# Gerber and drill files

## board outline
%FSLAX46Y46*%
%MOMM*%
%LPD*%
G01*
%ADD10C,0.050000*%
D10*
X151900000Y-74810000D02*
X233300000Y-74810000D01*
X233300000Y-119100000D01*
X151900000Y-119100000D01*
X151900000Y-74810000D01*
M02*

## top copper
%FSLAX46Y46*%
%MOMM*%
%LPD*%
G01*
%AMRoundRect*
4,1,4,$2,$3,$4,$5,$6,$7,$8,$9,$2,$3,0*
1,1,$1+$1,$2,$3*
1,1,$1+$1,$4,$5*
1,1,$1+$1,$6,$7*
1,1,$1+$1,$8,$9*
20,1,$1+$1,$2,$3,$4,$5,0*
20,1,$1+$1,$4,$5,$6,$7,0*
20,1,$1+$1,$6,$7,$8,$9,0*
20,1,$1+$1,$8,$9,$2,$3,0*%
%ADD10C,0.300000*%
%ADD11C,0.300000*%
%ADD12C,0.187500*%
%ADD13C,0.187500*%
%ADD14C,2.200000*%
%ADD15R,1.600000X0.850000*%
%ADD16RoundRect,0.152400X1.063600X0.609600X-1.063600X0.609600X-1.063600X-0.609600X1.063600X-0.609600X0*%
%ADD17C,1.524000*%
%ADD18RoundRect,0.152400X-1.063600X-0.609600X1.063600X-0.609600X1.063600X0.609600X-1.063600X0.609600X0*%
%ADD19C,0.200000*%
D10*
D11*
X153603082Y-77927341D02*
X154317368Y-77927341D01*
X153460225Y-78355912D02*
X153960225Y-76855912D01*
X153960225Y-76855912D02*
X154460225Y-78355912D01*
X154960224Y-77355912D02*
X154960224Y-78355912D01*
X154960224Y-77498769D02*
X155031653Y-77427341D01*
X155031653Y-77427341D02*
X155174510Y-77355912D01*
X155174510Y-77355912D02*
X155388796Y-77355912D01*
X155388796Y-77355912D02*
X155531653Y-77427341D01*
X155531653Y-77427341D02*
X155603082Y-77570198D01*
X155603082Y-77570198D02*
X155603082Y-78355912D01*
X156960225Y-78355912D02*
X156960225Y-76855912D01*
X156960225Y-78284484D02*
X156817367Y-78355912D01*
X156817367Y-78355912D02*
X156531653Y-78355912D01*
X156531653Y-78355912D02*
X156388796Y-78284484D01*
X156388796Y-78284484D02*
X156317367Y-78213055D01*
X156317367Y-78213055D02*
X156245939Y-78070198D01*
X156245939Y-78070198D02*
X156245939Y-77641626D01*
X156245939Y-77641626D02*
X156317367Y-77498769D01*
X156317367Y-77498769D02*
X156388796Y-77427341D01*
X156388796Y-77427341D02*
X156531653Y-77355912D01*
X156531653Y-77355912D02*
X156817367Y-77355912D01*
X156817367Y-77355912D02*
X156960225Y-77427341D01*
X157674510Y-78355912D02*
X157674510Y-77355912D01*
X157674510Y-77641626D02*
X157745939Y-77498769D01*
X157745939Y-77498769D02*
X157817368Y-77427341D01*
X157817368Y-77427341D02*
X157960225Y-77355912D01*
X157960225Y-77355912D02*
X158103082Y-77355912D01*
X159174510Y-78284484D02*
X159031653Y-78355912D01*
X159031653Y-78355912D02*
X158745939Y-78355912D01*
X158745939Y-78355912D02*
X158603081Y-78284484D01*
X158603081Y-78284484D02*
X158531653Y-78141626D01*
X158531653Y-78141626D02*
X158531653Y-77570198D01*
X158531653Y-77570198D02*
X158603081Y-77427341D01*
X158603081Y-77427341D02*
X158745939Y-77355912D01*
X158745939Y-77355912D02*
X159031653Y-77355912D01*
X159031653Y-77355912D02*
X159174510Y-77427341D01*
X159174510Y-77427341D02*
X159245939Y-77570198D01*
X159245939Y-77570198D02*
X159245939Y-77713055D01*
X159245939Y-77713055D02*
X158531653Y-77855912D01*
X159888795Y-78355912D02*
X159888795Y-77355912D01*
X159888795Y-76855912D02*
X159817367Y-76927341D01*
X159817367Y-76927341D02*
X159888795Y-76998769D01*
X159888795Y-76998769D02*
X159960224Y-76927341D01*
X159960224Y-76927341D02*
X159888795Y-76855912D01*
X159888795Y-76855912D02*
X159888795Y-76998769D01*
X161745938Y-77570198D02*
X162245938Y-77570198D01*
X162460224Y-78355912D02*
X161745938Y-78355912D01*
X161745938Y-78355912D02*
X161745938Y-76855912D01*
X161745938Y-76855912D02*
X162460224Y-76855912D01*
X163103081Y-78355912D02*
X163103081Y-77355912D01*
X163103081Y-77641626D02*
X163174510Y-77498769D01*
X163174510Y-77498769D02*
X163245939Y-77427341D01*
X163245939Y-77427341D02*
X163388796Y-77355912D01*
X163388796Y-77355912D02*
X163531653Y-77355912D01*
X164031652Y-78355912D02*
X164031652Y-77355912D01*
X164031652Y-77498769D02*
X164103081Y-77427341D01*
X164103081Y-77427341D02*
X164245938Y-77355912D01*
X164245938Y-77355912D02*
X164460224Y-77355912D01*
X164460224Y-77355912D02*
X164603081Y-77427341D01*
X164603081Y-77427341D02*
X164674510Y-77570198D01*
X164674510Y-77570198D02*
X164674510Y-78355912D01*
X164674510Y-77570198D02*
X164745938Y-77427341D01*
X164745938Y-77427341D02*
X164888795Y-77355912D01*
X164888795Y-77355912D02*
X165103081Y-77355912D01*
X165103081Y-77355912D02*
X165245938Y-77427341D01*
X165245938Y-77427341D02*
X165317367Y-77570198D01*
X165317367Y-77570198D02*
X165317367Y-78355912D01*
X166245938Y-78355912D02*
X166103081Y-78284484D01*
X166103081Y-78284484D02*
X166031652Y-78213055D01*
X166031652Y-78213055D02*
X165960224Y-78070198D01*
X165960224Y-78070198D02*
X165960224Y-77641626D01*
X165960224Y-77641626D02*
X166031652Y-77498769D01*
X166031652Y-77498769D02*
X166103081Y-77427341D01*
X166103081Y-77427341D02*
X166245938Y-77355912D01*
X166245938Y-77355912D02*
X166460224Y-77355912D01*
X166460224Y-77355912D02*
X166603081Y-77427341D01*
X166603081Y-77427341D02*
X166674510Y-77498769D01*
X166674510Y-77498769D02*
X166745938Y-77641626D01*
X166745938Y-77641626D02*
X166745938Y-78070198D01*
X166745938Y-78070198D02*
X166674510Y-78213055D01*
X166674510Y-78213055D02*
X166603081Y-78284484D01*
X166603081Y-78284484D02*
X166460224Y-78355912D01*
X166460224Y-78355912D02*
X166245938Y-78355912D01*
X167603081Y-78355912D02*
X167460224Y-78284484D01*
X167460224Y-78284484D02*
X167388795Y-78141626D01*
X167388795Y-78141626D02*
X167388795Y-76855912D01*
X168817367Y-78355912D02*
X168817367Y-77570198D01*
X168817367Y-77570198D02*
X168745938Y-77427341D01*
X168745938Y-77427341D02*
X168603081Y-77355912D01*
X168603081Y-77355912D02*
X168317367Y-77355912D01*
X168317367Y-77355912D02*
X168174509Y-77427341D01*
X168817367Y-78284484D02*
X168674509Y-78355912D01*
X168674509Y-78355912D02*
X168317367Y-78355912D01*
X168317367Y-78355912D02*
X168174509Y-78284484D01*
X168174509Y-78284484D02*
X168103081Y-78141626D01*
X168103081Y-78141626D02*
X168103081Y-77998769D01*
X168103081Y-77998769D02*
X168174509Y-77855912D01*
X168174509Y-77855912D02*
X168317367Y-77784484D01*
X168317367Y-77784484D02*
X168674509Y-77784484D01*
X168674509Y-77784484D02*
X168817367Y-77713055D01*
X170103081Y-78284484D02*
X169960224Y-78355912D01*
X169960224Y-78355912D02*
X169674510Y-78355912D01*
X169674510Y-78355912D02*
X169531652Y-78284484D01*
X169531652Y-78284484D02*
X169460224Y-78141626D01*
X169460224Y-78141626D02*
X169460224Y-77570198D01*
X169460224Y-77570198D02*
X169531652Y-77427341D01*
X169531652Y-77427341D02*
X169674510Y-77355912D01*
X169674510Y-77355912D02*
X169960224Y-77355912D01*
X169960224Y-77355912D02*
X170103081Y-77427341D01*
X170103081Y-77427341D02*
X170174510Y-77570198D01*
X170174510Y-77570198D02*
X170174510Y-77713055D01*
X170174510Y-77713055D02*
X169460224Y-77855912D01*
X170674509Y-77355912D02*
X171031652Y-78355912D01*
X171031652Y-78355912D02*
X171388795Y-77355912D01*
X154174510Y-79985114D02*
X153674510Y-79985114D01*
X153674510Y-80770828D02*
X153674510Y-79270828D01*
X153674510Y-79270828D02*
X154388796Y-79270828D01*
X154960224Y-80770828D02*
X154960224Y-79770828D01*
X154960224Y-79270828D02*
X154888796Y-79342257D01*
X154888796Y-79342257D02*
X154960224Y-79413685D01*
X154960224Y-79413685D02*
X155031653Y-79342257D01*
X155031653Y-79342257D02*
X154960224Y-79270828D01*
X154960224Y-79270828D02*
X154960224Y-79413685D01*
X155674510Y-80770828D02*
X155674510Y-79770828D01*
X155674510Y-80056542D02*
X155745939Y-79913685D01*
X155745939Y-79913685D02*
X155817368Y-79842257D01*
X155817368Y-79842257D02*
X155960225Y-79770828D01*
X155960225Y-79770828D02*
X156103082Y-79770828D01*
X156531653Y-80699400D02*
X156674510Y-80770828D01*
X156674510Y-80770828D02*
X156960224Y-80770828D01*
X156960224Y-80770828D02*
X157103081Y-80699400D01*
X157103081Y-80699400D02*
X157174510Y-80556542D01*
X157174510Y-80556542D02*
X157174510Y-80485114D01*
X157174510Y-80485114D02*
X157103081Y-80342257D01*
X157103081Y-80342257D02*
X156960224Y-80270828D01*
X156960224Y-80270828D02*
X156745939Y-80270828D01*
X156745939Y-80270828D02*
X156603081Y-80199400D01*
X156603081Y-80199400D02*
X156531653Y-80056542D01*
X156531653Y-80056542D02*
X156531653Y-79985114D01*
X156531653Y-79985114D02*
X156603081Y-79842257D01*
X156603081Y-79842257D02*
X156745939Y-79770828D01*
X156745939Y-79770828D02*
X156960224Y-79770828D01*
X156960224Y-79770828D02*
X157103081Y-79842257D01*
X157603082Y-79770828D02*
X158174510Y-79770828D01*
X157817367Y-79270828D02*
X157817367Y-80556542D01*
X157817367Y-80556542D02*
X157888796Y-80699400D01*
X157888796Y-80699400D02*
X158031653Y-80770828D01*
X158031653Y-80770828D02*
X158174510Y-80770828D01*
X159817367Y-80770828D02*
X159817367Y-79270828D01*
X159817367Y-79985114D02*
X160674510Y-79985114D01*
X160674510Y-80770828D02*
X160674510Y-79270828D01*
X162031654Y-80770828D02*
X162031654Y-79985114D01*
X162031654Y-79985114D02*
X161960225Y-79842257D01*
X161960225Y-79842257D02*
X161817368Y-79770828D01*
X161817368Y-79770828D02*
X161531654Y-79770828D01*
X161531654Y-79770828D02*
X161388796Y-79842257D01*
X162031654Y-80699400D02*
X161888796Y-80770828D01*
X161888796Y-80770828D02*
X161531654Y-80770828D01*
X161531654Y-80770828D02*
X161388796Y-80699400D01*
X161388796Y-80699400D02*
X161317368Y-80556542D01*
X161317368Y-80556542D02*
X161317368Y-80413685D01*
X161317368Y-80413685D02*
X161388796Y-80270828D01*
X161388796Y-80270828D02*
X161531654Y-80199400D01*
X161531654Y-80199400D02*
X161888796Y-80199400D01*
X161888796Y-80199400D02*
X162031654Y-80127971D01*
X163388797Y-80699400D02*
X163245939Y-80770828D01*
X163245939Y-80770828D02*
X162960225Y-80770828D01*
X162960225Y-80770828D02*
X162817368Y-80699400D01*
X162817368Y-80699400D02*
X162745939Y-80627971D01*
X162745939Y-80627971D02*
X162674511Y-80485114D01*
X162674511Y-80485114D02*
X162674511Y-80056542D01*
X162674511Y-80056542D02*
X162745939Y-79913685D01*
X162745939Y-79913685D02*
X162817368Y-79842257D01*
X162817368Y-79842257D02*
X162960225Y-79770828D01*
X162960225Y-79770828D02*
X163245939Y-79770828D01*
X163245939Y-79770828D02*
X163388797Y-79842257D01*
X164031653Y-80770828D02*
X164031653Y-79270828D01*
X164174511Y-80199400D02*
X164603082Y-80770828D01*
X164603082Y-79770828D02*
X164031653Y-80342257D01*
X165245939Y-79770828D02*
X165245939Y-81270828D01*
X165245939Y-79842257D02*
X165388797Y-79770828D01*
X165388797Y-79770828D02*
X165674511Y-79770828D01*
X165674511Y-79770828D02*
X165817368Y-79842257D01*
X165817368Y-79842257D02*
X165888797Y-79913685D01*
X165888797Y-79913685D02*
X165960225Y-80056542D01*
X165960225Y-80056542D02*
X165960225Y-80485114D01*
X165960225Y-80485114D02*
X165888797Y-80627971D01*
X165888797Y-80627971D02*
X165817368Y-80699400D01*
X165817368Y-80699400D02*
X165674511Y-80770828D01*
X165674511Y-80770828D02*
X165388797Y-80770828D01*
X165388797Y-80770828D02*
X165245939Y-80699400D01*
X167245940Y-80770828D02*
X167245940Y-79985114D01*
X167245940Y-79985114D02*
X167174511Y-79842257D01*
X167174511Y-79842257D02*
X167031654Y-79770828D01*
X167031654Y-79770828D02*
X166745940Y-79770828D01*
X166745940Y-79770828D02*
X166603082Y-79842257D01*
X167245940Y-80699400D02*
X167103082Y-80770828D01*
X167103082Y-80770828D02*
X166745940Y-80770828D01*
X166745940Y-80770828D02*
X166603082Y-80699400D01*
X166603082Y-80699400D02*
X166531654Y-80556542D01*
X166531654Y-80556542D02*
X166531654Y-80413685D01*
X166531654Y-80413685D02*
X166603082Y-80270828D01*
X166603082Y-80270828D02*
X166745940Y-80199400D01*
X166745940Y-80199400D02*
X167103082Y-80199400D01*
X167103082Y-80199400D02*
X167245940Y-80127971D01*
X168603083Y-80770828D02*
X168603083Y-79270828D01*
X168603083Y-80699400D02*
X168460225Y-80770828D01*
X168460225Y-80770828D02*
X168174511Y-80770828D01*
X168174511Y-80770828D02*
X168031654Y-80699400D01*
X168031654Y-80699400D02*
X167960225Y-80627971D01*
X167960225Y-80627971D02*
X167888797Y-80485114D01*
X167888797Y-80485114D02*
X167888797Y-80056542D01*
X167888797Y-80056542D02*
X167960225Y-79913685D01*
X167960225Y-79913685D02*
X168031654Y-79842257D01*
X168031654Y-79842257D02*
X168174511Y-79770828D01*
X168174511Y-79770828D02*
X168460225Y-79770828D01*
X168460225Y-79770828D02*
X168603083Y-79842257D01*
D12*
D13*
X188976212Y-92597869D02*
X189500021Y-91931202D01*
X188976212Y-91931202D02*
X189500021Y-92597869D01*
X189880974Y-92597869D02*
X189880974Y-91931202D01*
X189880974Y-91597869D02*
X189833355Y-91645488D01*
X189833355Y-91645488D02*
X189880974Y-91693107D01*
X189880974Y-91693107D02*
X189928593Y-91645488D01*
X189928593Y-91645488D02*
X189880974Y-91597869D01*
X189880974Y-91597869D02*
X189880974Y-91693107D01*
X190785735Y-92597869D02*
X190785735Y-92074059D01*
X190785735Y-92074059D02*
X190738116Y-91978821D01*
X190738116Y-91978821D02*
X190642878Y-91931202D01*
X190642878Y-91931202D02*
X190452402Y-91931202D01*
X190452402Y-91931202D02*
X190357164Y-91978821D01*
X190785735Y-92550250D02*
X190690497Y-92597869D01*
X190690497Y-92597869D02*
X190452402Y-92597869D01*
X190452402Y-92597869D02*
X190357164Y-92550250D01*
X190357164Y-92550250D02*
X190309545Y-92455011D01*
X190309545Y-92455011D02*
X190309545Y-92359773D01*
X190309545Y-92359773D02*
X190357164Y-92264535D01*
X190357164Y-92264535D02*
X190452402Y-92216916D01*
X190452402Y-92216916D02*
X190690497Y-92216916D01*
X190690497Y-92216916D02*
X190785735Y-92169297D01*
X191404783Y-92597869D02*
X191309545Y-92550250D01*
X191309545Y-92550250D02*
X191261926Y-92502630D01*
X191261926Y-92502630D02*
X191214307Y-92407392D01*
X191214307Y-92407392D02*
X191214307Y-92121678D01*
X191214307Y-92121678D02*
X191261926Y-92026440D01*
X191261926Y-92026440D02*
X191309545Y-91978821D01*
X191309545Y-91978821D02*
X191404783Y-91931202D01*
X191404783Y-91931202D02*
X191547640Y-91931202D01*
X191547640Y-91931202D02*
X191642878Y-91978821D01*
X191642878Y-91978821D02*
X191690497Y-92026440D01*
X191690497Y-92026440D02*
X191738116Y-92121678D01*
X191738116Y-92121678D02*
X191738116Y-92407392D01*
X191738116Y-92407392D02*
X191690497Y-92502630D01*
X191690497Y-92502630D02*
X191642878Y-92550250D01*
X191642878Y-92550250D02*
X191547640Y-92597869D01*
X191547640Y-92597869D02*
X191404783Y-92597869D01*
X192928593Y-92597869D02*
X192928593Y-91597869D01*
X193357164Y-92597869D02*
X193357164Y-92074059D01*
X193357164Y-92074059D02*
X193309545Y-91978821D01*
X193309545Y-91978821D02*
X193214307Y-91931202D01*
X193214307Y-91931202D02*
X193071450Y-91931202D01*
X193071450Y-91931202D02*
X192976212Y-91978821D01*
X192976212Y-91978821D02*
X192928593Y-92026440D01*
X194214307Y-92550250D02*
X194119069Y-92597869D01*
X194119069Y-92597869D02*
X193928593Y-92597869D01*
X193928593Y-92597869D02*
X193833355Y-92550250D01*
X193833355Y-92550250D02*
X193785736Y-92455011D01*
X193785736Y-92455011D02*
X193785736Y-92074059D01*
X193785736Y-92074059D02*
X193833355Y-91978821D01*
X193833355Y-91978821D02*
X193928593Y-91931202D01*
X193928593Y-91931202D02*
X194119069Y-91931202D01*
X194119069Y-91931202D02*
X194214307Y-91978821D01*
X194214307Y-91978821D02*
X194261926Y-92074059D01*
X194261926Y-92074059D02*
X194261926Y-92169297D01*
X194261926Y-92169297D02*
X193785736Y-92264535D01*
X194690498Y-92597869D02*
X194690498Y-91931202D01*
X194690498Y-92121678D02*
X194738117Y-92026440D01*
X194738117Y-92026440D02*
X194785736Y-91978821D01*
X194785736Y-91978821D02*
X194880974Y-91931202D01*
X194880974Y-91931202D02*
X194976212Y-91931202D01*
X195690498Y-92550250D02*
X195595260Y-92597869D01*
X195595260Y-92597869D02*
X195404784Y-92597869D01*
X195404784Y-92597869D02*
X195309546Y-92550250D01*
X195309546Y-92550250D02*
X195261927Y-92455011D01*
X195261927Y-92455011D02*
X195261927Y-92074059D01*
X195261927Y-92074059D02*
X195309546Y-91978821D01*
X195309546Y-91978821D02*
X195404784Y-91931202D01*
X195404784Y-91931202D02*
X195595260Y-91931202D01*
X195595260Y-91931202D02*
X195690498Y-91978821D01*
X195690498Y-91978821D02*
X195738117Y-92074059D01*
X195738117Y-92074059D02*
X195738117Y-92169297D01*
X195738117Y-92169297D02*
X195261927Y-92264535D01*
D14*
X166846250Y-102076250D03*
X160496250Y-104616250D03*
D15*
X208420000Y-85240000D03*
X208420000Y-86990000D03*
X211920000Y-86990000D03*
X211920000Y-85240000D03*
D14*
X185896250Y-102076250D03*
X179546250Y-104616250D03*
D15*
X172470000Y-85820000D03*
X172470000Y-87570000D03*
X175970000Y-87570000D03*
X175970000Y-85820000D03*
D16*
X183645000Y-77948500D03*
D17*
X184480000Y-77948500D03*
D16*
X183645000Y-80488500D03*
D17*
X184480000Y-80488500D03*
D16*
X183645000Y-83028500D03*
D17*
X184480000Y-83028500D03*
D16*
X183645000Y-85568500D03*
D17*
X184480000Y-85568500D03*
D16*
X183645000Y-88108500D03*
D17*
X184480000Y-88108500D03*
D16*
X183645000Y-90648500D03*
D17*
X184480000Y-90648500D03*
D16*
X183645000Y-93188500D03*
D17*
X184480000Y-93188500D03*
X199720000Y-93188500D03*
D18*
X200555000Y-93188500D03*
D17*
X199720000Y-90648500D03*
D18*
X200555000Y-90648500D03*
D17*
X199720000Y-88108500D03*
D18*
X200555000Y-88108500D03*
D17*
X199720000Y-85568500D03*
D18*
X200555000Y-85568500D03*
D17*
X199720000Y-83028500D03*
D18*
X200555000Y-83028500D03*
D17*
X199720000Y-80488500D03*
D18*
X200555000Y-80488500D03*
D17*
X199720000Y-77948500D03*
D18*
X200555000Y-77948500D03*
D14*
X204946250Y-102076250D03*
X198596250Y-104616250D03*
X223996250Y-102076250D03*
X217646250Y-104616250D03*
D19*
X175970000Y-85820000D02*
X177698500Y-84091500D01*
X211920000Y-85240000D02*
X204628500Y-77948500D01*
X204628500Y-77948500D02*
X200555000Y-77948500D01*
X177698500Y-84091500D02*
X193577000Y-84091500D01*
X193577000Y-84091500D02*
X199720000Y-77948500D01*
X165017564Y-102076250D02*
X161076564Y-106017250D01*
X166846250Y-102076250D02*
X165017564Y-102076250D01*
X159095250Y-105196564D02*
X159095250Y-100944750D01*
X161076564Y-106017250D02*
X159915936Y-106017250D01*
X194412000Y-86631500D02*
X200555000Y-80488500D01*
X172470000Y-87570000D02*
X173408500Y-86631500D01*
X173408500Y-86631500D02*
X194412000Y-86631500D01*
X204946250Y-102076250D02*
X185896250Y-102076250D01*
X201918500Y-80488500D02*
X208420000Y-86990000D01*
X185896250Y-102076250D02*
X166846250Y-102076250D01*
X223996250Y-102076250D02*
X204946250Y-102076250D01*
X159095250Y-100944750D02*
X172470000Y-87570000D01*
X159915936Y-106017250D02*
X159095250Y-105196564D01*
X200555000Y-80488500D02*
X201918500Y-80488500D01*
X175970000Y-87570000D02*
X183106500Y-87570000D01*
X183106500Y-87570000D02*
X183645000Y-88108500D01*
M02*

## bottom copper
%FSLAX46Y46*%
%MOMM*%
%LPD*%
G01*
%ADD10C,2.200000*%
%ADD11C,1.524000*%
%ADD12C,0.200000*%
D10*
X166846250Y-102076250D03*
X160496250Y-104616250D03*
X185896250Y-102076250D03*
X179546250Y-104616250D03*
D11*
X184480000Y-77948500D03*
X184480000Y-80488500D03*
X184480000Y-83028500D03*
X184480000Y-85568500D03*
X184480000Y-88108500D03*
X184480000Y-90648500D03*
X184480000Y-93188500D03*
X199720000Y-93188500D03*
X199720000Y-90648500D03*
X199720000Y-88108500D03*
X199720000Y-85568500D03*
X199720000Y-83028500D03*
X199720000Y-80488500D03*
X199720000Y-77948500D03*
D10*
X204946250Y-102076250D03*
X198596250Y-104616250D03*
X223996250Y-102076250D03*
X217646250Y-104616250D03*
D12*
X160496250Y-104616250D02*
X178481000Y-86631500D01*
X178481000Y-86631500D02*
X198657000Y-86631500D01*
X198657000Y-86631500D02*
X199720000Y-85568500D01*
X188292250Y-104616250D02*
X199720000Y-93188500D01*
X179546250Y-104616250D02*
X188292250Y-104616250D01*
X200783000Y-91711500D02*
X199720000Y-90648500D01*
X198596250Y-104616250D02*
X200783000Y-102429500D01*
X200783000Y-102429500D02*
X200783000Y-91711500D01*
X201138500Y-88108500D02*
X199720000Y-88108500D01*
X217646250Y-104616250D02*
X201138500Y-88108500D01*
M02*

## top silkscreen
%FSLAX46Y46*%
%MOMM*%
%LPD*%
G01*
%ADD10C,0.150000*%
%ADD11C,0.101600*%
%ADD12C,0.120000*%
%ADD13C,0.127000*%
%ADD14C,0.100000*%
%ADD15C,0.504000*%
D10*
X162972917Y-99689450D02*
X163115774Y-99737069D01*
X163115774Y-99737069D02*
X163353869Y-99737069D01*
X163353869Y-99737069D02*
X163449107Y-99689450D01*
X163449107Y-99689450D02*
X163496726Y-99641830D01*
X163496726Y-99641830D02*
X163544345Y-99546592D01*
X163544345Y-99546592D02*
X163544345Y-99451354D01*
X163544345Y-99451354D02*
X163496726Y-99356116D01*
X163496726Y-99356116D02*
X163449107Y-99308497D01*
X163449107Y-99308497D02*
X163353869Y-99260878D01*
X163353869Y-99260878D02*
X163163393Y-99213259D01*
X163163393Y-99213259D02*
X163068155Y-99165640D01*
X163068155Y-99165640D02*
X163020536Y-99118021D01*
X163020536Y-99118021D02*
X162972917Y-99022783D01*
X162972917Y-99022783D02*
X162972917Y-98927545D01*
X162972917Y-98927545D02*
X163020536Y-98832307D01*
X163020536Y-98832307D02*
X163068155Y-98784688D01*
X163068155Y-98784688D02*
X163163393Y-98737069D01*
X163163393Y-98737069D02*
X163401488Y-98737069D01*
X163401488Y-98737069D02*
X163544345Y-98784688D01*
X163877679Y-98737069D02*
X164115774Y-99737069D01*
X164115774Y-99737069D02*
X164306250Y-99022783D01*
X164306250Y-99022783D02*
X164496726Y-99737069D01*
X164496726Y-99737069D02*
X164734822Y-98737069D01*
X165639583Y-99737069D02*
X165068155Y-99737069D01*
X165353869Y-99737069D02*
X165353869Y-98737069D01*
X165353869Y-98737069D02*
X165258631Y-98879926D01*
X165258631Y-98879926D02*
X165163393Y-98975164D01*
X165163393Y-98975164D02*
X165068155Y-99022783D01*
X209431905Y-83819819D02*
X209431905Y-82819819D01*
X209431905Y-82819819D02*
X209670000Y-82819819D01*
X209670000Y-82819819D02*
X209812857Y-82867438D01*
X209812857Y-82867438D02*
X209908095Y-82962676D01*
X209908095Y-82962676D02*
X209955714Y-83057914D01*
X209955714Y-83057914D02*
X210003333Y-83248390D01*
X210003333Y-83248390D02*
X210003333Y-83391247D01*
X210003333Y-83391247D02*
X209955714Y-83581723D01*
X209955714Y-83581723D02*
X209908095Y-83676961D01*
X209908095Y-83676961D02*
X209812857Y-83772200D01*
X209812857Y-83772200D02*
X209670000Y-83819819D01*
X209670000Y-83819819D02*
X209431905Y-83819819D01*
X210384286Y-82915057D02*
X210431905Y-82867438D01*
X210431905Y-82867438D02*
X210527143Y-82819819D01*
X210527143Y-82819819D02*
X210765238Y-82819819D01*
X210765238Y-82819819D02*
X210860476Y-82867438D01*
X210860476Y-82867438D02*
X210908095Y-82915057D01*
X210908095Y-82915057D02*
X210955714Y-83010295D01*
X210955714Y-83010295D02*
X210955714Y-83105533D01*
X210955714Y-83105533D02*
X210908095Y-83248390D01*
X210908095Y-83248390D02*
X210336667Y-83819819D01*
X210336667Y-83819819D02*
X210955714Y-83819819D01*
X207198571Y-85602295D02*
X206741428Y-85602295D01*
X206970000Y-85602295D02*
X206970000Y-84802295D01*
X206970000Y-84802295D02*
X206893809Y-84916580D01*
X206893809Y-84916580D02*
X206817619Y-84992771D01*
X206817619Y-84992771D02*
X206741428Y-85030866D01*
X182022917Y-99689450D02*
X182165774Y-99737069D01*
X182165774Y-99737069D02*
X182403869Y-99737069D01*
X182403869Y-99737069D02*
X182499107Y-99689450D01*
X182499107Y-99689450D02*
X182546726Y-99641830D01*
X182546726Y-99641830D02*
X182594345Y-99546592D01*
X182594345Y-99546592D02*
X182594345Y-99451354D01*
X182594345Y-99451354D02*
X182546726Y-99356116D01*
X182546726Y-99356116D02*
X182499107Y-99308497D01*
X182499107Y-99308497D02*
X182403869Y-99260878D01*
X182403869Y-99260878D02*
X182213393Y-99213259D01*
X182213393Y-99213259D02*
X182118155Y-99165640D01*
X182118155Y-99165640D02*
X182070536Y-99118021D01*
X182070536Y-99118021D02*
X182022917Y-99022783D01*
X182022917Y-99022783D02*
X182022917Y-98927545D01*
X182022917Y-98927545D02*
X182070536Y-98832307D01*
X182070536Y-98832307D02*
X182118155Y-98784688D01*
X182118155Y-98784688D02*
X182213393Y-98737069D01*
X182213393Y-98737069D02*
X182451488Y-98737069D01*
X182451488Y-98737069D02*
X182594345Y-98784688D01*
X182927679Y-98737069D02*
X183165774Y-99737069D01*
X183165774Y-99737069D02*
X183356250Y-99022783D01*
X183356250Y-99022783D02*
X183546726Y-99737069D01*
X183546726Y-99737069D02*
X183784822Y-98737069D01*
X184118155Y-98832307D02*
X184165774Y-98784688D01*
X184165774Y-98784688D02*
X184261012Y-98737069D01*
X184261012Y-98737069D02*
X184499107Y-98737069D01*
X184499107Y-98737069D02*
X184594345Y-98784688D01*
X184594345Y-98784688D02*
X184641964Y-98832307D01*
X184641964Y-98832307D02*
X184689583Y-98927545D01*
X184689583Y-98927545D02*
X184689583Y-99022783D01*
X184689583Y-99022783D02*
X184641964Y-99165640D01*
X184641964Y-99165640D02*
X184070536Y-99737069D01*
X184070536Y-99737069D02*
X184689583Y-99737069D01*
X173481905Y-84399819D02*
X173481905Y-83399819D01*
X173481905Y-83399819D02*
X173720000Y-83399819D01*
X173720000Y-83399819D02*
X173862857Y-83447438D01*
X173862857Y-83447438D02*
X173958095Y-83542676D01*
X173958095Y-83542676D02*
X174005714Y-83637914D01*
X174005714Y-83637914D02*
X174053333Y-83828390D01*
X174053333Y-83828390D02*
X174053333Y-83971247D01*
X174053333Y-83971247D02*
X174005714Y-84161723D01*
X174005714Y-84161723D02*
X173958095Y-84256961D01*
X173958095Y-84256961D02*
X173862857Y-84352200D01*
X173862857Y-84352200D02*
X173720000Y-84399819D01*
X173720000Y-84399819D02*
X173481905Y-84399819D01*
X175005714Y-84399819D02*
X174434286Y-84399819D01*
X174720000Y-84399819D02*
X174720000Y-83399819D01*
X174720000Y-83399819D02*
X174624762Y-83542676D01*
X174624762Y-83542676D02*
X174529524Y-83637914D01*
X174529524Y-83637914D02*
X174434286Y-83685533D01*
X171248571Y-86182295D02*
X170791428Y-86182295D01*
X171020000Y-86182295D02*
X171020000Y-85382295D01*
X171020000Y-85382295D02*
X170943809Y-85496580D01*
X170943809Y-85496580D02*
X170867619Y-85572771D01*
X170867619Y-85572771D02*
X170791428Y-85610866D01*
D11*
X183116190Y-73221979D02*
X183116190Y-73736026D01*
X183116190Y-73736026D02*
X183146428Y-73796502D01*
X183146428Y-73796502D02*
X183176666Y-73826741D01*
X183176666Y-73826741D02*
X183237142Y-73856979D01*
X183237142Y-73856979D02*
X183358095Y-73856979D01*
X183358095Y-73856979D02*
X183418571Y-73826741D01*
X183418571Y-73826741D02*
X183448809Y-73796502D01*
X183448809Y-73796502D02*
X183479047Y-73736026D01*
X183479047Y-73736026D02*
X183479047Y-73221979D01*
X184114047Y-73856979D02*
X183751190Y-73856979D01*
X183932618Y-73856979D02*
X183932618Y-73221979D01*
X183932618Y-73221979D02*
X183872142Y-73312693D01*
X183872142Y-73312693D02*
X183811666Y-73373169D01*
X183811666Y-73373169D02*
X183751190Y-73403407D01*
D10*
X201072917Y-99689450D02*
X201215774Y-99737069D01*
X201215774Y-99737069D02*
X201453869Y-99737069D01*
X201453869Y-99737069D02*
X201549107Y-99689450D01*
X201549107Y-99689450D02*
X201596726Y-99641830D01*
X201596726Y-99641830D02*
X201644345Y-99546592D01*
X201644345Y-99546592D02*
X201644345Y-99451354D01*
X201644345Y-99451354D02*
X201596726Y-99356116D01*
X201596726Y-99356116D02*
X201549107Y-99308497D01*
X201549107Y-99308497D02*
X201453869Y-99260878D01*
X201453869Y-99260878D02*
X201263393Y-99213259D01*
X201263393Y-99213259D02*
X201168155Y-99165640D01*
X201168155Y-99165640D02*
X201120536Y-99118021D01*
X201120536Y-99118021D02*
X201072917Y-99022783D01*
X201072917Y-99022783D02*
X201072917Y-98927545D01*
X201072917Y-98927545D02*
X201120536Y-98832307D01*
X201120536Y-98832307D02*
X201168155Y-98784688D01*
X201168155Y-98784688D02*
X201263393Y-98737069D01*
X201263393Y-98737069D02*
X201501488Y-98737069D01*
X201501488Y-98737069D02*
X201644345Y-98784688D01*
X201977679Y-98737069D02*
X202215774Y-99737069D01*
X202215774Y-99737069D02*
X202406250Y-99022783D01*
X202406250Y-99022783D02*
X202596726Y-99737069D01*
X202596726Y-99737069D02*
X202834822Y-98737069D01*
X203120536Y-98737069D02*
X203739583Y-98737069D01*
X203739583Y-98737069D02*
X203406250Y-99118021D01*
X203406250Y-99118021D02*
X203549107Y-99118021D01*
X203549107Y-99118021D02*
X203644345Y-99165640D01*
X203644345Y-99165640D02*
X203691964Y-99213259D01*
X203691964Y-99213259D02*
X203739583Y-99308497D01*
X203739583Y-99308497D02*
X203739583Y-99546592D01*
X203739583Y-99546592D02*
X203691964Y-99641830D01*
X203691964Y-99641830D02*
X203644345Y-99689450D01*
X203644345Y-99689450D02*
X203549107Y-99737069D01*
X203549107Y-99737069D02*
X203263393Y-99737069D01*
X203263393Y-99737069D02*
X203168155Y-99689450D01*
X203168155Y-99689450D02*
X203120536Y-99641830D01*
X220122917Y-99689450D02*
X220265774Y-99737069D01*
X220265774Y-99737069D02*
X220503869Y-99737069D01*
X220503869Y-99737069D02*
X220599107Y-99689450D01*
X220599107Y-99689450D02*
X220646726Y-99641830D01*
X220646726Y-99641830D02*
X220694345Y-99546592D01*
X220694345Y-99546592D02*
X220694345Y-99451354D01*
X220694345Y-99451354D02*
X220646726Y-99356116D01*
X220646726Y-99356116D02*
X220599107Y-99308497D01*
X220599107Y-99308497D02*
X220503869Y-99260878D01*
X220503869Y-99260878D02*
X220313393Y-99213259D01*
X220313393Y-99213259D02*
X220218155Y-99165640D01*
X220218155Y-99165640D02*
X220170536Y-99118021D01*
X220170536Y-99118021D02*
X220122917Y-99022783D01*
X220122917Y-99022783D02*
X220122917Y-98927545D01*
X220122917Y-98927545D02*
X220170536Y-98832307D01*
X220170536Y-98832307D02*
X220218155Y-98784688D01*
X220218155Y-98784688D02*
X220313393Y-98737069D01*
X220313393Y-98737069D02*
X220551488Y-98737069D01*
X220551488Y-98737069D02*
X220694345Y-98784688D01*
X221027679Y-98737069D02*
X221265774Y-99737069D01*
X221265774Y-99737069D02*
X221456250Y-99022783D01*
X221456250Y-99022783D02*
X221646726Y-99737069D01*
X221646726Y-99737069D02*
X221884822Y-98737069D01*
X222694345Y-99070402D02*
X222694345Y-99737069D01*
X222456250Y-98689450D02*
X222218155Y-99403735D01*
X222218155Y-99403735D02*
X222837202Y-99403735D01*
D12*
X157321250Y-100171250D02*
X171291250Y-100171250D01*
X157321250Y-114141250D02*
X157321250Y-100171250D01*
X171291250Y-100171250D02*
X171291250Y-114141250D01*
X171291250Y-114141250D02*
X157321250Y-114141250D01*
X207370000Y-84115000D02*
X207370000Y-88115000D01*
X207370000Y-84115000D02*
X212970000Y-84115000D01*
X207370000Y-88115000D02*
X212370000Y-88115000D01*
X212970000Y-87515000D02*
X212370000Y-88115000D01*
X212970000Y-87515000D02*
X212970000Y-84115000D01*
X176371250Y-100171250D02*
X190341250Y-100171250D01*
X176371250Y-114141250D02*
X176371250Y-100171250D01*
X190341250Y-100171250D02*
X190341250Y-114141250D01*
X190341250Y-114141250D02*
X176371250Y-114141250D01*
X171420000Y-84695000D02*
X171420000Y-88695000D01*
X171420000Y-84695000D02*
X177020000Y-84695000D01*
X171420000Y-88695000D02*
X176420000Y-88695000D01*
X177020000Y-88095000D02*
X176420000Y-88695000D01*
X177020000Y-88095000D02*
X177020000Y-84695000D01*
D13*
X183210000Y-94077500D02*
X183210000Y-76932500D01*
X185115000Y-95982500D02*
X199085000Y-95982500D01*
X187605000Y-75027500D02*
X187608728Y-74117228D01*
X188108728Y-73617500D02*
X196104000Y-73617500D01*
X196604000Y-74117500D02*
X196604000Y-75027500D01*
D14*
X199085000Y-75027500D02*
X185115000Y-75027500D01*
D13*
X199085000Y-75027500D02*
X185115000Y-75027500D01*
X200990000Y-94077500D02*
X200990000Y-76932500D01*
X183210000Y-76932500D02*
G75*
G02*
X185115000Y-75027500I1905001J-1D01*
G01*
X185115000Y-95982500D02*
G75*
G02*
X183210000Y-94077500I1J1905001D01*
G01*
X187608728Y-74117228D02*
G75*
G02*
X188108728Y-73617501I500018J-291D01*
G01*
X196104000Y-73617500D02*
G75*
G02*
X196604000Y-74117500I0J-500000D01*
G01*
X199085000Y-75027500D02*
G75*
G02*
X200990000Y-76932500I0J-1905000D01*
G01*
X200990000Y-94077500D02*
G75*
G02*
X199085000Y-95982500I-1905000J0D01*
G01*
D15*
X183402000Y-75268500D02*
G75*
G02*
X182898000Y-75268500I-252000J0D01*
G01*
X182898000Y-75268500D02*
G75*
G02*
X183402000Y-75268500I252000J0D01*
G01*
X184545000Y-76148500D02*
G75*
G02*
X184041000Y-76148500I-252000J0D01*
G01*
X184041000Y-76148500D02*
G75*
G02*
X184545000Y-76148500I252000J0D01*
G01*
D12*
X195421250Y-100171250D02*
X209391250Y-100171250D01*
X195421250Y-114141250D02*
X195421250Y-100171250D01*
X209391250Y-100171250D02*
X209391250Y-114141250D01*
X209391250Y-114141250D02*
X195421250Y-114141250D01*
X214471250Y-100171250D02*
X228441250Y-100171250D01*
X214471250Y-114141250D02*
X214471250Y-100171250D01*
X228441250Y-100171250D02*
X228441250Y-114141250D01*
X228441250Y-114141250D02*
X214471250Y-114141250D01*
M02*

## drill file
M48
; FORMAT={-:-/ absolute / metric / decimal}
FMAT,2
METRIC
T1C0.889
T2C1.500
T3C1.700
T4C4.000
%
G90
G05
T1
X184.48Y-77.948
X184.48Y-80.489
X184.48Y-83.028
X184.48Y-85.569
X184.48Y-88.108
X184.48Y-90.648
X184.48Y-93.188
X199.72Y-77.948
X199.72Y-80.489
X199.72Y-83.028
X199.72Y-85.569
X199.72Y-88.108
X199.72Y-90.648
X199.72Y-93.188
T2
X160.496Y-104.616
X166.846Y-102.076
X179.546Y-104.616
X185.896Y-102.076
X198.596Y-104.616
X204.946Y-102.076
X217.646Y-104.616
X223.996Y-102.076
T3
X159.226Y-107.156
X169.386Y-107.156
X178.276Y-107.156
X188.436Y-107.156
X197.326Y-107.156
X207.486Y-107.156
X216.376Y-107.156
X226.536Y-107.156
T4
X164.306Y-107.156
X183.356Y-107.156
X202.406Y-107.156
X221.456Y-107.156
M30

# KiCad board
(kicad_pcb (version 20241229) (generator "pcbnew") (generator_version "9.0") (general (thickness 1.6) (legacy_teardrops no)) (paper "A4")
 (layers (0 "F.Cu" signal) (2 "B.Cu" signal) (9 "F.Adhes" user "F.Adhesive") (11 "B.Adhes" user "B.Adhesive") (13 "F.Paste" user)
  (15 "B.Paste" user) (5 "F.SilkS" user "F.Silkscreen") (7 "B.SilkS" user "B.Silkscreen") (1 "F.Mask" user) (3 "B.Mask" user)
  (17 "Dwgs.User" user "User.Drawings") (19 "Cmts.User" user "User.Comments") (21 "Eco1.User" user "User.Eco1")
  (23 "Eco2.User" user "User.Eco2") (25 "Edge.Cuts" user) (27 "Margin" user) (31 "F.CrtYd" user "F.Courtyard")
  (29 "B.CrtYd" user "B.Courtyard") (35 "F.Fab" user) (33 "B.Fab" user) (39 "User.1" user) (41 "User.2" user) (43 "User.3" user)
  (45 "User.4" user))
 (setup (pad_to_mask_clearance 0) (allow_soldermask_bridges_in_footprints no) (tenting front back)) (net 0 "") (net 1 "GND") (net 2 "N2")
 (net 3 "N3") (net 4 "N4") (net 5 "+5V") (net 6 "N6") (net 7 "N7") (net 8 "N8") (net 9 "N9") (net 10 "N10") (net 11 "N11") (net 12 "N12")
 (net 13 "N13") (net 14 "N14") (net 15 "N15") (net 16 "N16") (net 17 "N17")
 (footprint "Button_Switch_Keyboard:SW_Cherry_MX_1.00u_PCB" (layer "F.Cu") (at 166.84625 102.07625)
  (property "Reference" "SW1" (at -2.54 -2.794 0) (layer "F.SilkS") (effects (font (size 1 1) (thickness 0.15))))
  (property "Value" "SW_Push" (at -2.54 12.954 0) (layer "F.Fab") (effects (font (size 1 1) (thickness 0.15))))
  (fp_line (start -9.525 -1.905) (end 4.445 -1.905) (stroke (width 0.12) (type solid)) (layer "F.SilkS"))
  (fp_line (start -9.525 12.065) (end -9.525 -1.905) (stroke (width 0.12) (type solid)) (layer "F.SilkS"))
  (fp_line (start 4.445 -1.905) (end 4.445 12.065) (stroke (width 0.12) (type solid)) (layer "F.SilkS"))
  (fp_line (start 4.445 12.065) (end -9.525 12.065) (stroke (width 0.12) (type solid)) (layer "F.SilkS"))
  (pad "" np_thru_hole circle (at -7.62 5.08) (size 1.7 1.7) (drill 1.7) (layers "*.Cu" "*.Mask"))
  (pad "" np_thru_hole circle (at -2.54 5.08) (size 4 4) (drill 4) (layers "*.Cu" "*.Mask"))
  (pad "" np_thru_hole circle (at 2.54 5.08) (size 1.7 1.7) (drill 1.7) (layers "*.Cu" "*.Mask"))
  (pad "1" thru_hole circle (at 0 0) (size 2.2 2.2) (drill 1.5) (layers "*.Cu" "*.Mask") (remove_unused_layers no) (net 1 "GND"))
  (pad "2" thru_hole circle (at -6.35 2.54) (size 2.2 2.2) (drill 1.5) (layers "*.Cu" "*.Mask") (remove_unused_layers no) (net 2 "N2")))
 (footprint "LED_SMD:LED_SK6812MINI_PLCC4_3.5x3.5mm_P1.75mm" (layer "F.Cu") (at 210.17 86.115)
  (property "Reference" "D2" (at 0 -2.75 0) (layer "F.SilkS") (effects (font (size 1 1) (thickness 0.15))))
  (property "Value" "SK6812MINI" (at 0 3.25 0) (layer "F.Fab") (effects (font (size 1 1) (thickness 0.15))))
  (fp_line (start -2.8 -2) (end -2.8 2) (stroke (width 0.12) (type default)) (layer "F.SilkS"))
  (fp_line (start -2.8 -2) (end 2.8 -2) (stroke (width 0.12) (type solid)) (layer "F.SilkS"))
  (fp_line (start -2.8 2) (end 2.2 2) (stroke (width 0.12) (type solid)) (layer "F.SilkS"))
  (fp_line (start 2.8 1.4) (end 2.2 2) (stroke (width 0.12) (type default)) (layer "F.SilkS"))
  (fp_line (start 2.8 1.4) (end 2.8 -2) (stroke (width 0.12) (type solid)) (layer "F.SilkS"))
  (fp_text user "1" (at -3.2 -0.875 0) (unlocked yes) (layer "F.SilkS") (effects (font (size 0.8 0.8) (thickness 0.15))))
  (pad "1" smd rect (at -1.75 -0.875) (size 1.6 0.85) (layers "F.Cu" "F.Mask" "F.Paste") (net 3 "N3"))
  (pad "2" smd rect (at -1.75 0.875) (size 1.6 0.85) (layers "F.Cu" "F.Mask" "F.Paste") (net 1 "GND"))
  (pad "3" smd rect (at 1.75 0.875) (size 1.6 0.85) (layers "F.Cu" "F.Mask" "F.Paste") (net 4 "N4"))
  (pad "4" smd rect (at 1.75 -0.875) (size 1.6 0.85) (layers "F.Cu" "F.Mask" "F.Paste") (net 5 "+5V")))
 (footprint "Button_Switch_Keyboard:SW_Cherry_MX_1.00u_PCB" (layer "F.Cu") (at 185.89625 102.07625)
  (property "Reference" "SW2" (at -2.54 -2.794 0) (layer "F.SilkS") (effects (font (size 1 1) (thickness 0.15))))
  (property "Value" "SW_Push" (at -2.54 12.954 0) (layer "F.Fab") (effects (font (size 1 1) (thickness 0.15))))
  (fp_line (start -9.525 -1.905) (end 4.445 -1.905) (stroke (width 0.12) (type solid)) (layer "F.SilkS"))
  (fp_line (start -9.525 12.065) (end -9.525 -1.905) (stroke (width 0.12) (type solid)) (layer "F.SilkS"))
  (fp_line (start 4.445 -1.905) (end 4.445 12.065) (stroke (width 0.12) (type solid)) (layer "F.SilkS"))
  (fp_line (start 4.445 12.065) (end -9.525 12.065) (stroke (width 0.12) (type solid)) (layer "F.SilkS"))
  (pad "" np_thru_hole circle (at -7.62 5.08) (size 1.7 1.7) (drill 1.7) (layers "*.Cu" "*.Mask"))
  (pad "" np_thru_hole circle (at -2.54 5.08) (size 4 4) (drill 4) (layers "*.Cu" "*.Mask"))
  (pad "" np_thru_hole circle (at 2.54 5.08) (size 1.7 1.7) (drill 1.7) (layers "*.Cu" "*.Mask"))
  (pad "1" thru_hole circle (at 0 0) (size 2.2 2.2) (drill 1.5) (layers "*.Cu" "*.Mask") (remove_unused_layers no) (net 1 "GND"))
  (pad "2" thru_hole circle (at -6.35 2.54) (size 2.2 2.2) (drill 1.5) (layers "*.Cu" "*.Mask") (remove_unused_layers no) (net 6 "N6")))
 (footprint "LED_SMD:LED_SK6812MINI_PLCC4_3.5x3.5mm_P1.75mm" (layer "F.Cu") (at 174.22 86.695)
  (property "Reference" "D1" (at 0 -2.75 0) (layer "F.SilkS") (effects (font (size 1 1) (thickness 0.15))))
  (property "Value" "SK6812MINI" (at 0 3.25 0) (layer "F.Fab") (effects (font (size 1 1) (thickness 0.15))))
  (fp_line (start -2.8 -2) (end -2.8 2) (stroke (width 0.12) (type default)) (layer "F.SilkS"))
  (fp_line (start -2.8 -2) (end 2.8 -2) (stroke (width 0.12) (type solid)) (layer "F.SilkS"))
  (fp_line (start -2.8 2) (end 2.2 2) (stroke (width 0.12) (type solid)) (layer "F.SilkS"))
  (fp_line (start 2.8 1.4) (end 2.2 2) (stroke (width 0.12) (type default)) (layer "F.SilkS"))
  (fp_line (start 2.8 1.4) (end 2.8 -2) (stroke (width 0.12) (type solid)) (layer "F.SilkS"))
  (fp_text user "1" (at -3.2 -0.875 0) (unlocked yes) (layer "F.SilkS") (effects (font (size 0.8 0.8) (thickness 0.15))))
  (pad "1" smd rect (at -1.75 -0.875) (size 1.6 0.85) (layers "F.Cu" "F.Mask" "F.Paste") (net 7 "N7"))
  (pad "2" smd rect (at -1.75 0.875) (size 1.6 0.85) (layers "F.Cu" "F.Mask" "F.Paste") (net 1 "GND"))
  (pad "3" smd rect (at 1.75 0.875) (size 1.6 0.85) (layers "F.Cu" "F.Mask" "F.Paste") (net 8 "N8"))
  (pad "4" smd rect (at 1.75 -0.875) (size 1.6 0.85) (layers "F.Cu" "F.Mask" "F.Paste") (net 5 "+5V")))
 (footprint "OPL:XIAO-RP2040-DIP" (layer "F.Cu") (at 192.1 85.5685)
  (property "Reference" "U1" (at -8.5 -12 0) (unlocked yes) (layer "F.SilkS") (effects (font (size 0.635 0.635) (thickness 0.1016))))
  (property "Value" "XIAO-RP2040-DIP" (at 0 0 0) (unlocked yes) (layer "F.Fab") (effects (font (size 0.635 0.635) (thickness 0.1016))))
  (fp_line (start -8.89 8.509) (end -8.89 -8.636) (stroke (width 0.127) (type solid)) (layer "F.SilkS"))
  (fp_line (start -6.985 10.414) (end 6.985 10.414) (stroke (width 0.127) (type solid)) (layer "F.SilkS"))
  (fp_line (start -4.495 -10.541) (end -4.491272 -11.451272) (stroke (width 0.127) (type solid)) (layer "F.SilkS"))
  (fp_line (start -3.991272 -11.951) (end 4.004 -11.951) (stroke (width 0.127) (type solid)) (layer "F.SilkS"))
  (fp_line (start 4.504 -11.451) (end 4.504 -10.541) (stroke (width 0.127) (type solid)) (layer "F.SilkS"))
  (fp_line (start 6.985 -10.541) (end -6.985 -10.541) (stroke (width 0.1) (type solid)) (layer "F.SilkS"))
  (fp_line (start 6.985 -10.541) (end -6.985 -10.541) (stroke (width 0.127) (type solid)) (layer "F.SilkS"))
  (fp_line (start 8.89 8.509) (end 8.89 -8.636) (stroke (width 0.127) (type solid)) (layer "F.SilkS"))
  (fp_arc (start -8.89 -8.636) (mid -8.332038 -9.983038) (end -6.985 -10.541) (stroke (width 0.127) (type solid)) (layer "F.SilkS"))
  (fp_arc (start -6.985 10.414) (mid -8.332038 9.856038) (end -8.89 8.509) (stroke (width 0.127) (type solid)) (layer "F.SilkS"))
  (fp_arc (start -4.491272 -11.451272) (mid -4.344728 -11.80464) (end -3.991272 -11.951) (stroke (width 0.127) (type default))
   (layer "F.SilkS"))
  (fp_arc (start 4.004 -11.951) (mid 4.357553 -11.804553) (end 4.504 -11.451) (stroke (width 0.127) (type default)) (layer "F.SilkS"))
  (fp_arc (start 6.985 -10.541) (mid 8.332038 -9.983038) (end 8.89 -8.636) (stroke (width 0.127) (type solid)) (layer "F.SilkS"))
  (fp_arc (start 8.89 8.509) (mid 8.332038 9.856038) (end 6.985 10.414) (stroke (width 0.127) (type solid)) (layer "F.SilkS"))
  (fp_circle (center -8.95 -10.3) (end -8.95 -10.554) (stroke (width 0.5) (type solid)) (fill yes) (layer "F.SilkS"))
  (fp_circle (center -7.807 -9.42) (end -7.807 -9.674) (stroke (width 0.5) (type solid)) (fill yes) (layer "F.SilkS"))
  (pad "1" smd roundrect (at -8.455 -7.62 180) (size 2.432 1.524) (layers "F.Cu" "F.Mask") (roundrect_rratio 0.1) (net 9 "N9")
   (thermal_bridge_angle 45))
  (pad "1" thru_hole circle (at -7.62 -7.62 180) (size 1.524 1.524) (drill 0.889) (layers "*.Cu" "*.Mask") (remove_unused_layers no)
   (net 9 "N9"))
  (pad "2" smd roundrect (at -8.455 -5.08 180) (size 2.432 1.524) (layers "F.Cu" "F.Mask") (roundrect_rratio 0.1) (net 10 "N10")
   (thermal_bridge_angle 45))
  (pad "2" thru_hole circle (at -7.62 -5.08 180) (size 1.524 1.524) (drill 0.889) (layers "*.Cu" "*.Mask") (remove_unused_layers no)
   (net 10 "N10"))
  (pad "3" smd roundrect (at -8.455 -2.54 180) (size 2.432 1.524) (layers "F.Cu" "F.Mask") (roundrect_rratio 0.1) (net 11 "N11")
   (thermal_bridge_angle 45))
  (pad "3" thru_hole circle (at -7.62 -2.54 180) (size 1.524 1.524) (drill 0.889) (layers "*.Cu" "*.Mask") (remove_unused_layers no)
   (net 11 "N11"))
  (pad "4" smd roundrect (at -8.455 0 180) (size 2.432 1.524) (layers "F.Cu" "F.Mask") (roundrect_rratio 0.1) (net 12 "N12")
   (thermal_bridge_angle 45))
  (pad "4" thru_hole circle (at -7.62 0 180) (size 1.524 1.524) (drill 0.889) (layers "*.Cu" "*.Mask") (remove_unused_layers no)
   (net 12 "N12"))
  (pad "5" smd roundrect (at -8.455 2.54 180) (size 2.432 1.524) (layers "F.Cu" "F.Mask") (roundrect_rratio 0.1) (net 8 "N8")
   (thermal_bridge_angle 45))
  (pad "5" thru_hole circle (at -7.62 2.54 180) (size 1.524 1.524) (drill 0.889) (layers "*.Cu" "*.Mask") (remove_unused_layers no)
   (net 8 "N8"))
  (pad "6" smd roundrect (at -8.455 5.08 180) (size 2.432 1.524) (layers "F.Cu" "F.Mask") (roundrect_rratio 0.1) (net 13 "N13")
   (thermal_bridge_angle 45))
  (pad "6" thru_hole circle (at -7.62 5.08 180) (size 1.524 1.524) (drill 0.889) (layers "*.Cu" "*.Mask") (remove_unused_layers no)
   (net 13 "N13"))
  (pad "7" smd roundrect (at -8.455 7.62 180) (size 2.432 1.524) (layers "F.Cu" "F.Mask") (roundrect_rratio 0.1) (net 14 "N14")
   (thermal_bridge_angle 45))
  (pad "7" thru_hole circle (at -7.62 7.62 180) (size 1.524 1.524) (drill 0.889) (layers "*.Cu" "*.Mask") (remove_unused_layers no)
   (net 14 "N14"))
  (pad "8" thru_hole circle (at 7.62 7.62) (size 1.524 1.524) (drill 0.889) (layers "*.Cu" "*.Mask") (remove_unused_layers no) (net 6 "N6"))
  (pad "8" smd roundrect (at 8.455 7.62) (size 2.432 1.524) (layers "F.Cu" "F.Mask") (roundrect_rratio 0.1) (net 6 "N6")
   (thermal_bridge_angle 45))
  (pad "9" thru_hole circle (at 7.62 5.08) (size 1.524 1.524) (drill 0.889) (layers "*.Cu" "*.Mask") (remove_unused_layers no)
   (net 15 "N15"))
  (pad "9" smd roundrect (at 8.455 5.08) (size 2.432 1.524) (layers "F.Cu" "F.Mask") (roundrect_rratio 0.1) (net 15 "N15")
   (thermal_bridge_angle 45))
  (pad "10" thru_hole circle (at 7.62 2.54) (size 1.524 1.524) (drill 0.889) (layers "*.Cu" "*.Mask") (remove_unused_layers no)
   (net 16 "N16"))
  (pad "10" smd roundrect (at 8.455 2.54) (size 2.432 1.524) (layers "F.Cu" "F.Mask") (roundrect_rratio 0.1) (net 16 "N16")
   (thermal_bridge_angle 45))
  (pad "11" thru_hole circle (at 7.62 0) (size 1.524 1.524) (drill 0.889) (layers "*.Cu" "*.Mask") (remove_unused_layers no) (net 2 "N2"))
  (pad "11" smd roundrect (at 8.455 0) (size 2.432 1.524) (layers "F.Cu" "F.Mask") (roundrect_rratio 0.1) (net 2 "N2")
   (thermal_bridge_angle 45))
  (pad "12" thru_hole circle (at 7.62 -2.54) (size 1.524 1.524) (drill 0.889) (layers "*.Cu" "*.Mask") (remove_unused_layers no)
   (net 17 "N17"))
  (pad "12" smd roundrect (at 8.455 -2.54) (size 2.432 1.524) (layers "F.Cu" "F.Mask") (roundrect_rratio 0.1) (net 17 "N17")
   (thermal_bridge_angle 45))
  (pad "13" thru_hole circle (at 7.62 -5.08) (size 1.524 1.524) (drill 0.889) (layers "*.Cu" "*.Mask") (remove_unused_layers no)
   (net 1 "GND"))
  (pad "13" smd roundrect (at 8.455 -5.08) (size 2.432 1.524) (layers "F.Cu" "F.Mask") (roundrect_rratio 0.1) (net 1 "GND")
   (thermal_bridge_angle 45))
  (pad "14" thru_hole circle (at 7.62 -7.62) (size 1.524 1.524) (drill 0.889) (layers "*.Cu" "*.Mask") (remove_unused_layers no)
   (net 5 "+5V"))
  (pad "14" smd roundrect (at 8.455 -7.62) (size 2.432 1.524) (layers "F.Cu" "F.Mask") (roundrect_rratio 0.1) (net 5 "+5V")
   (thermal_bridge_angle 45)))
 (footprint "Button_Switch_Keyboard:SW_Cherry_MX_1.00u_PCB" (layer "F.Cu") (at 204.94625 102.07625)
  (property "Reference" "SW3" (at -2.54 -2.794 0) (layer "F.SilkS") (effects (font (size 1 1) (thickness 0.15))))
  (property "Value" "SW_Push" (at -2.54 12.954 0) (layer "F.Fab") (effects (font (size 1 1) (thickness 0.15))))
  (fp_line (start -9.525 -1.905) (end 4.445 -1.905) (stroke (width 0.12) (type solid)) (layer "F.SilkS"))
  (fp_line (start -9.525 12.065) (end -9.525 -1.905) (stroke (width 0.12) (type solid)) (layer "F.SilkS"))
  (fp_line (start 4.445 -1.905) (end 4.445 12.065) (stroke (width 0.12) (type solid)) (layer "F.SilkS"))
  (fp_line (start 4.445 12.065) (end -9.525 12.065) (stroke (width 0.12) (type solid)) (layer "F.SilkS"))
  (pad "" np_thru_hole circle (at -7.62 5.08) (size 1.7 1.7) (drill 1.7) (layers "*.Cu" "*.Mask"))
  (pad "" np_thru_hole circle (at -2.54 5.08) (size 4 4) (drill 4) (layers "*.Cu" "*.Mask"))
  (pad "" np_thru_hole circle (at 2.54 5.08) (size 1.7 1.7) (drill 1.7) (layers "*.Cu" "*.Mask"))
  (pad "1" thru_hole circle (at 0 0) (size 2.2 2.2) (drill 1.5) (layers "*.Cu" "*.Mask") (remove_unused_layers no) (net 1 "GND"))
  (pad "2" thru_hole circle (at -6.35 2.54) (size 2.2 2.2) (drill 1.5) (layers "*.Cu" "*.Mask") (remove_unused_layers no) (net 15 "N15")))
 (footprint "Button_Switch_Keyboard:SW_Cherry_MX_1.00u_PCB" (layer "F.Cu") (at 223.99625 102.07625)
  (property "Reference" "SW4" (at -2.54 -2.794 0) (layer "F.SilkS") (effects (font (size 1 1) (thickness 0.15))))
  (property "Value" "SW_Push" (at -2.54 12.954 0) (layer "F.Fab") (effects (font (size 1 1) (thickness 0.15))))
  (fp_line (start -9.525 -1.905) (end 4.445 -1.905) (stroke (width 0.12) (type solid)) (layer "F.SilkS"))
  (fp_line (start -9.525 12.065) (end -9.525 -1.905) (stroke (width 0.12) (type solid)) (layer "F.SilkS"))
  (fp_line (start 4.445 -1.905) (end 4.445 12.065) (stroke (width 0.12) (type solid)) (layer "F.SilkS"))
  (fp_line (start 4.445 12.065) (end -9.525 12.065) (stroke (width 0.12) (type solid)) (layer "F.SilkS"))
  (pad "" np_thru_hole circle (at -7.62 5.08) (size 1.7 1.7) (drill 1.7) (layers "*.Cu" "*.Mask"))
  (pad "" np_thru_hole circle (at -2.54 5.08) (size 4 4) (drill 4) (layers "*.Cu" "*.Mask"))
  (pad "" np_thru_hole circle (at 2.54 5.08) (size 1.7 1.7) (drill 1.7) (layers "*.Cu" "*.Mask"))
  (pad "1" thru_hole circle (at 0 0) (size 2.2 2.2) (drill 1.5) (layers "*.Cu" "*.Mask") (remove_unused_layers no) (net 1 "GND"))
  (pad "2" thru_hole circle (at -6.35 2.54) (size 2.2 2.2) (drill 1.5) (layers "*.Cu" "*.Mask") (remove_unused_layers no) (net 16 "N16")))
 (gr_rect (start 151.9 74.81) (end 233.3 119.1) (stroke (width 0.05) (type default)) (fill no) (layer "Edge.Cuts"))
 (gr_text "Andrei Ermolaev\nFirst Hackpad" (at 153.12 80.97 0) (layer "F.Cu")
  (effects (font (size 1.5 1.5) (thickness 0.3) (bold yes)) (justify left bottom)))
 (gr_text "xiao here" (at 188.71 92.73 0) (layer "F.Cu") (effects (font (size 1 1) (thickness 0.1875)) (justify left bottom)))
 (segment (start 175.97 85.82) (end 177.6985 84.0915) (width 0.2) (layer "F.Cu") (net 5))
 (segment (start 211.92 85.24) (end 204.6285 77.9485) (width 0.2) (layer "F.Cu") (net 5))
 (segment (start 204.6285 77.9485) (end 200.555 77.9485) (width 0.2) (layer "F.Cu") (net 5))
 (segment (start 177.6985 84.0915) (end 193.577 84.0915) (width 0.2) (layer "F.Cu") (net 5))
 (segment (start 193.577 84.0915) (end 199.72 77.9485) (width 0.2) (layer "F.Cu") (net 5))
 (segment (start 165.017564 102.07625) (end 161.076564 106.01725) (width 0.2) (layer "F.Cu") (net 1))
 (segment (start 166.84625 102.07625) (end 165.017564 102.07625) (width 0.2) (layer "F.Cu") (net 1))
 (segment (start 159.09525 105.196564) (end 159.09525 100.94475) (width 0.2) (layer "F.Cu") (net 1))
 (segment (start 161.076564 106.01725) (end 159.915936 106.01725) (width 0.2) (layer "F.Cu") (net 1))
 (segment (start 194.412 86.6315) (end 200.555 80.4885) (width 0.2) (layer "F.Cu") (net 1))
 (segment (start 172.47 87.57) (end 173.4085 86.6315) (width 0.2) (layer "F.Cu") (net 1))
 (segment (start 173.4085 86.6315) (end 194.412 86.6315) (width 0.2) (layer "F.Cu") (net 1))
 (segment (start 204.94625 102.07625) (end 185.89625 102.07625) (width 0.2) (layer "F.Cu") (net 1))
 (segment (start 201.9185 80.4885) (end 208.42 86.99) (width 0.2) (layer "F.Cu") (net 1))
 (segment (start 185.89625 102.07625) (end 166.84625 102.07625) (width 0.2) (layer "F.Cu") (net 1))
 (segment (start 223.99625 102.07625) (end 204.94625 102.07625) (width 0.2) (layer "F.Cu") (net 1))
 (segment (start 159.09525 100.94475) (end 172.47 87.57) (width 0.2) (layer "F.Cu") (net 1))
 (segment (start 159.915936 106.01725) (end 159.09525 105.196564) (width 0.2) (layer "F.Cu") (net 1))
 (segment (start 200.555 80.4885) (end 201.9185 80.4885) (width 0.2) (layer "F.Cu") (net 1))
 (segment (start 175.97 87.57) (end 183.1065 87.57) (width 0.2) (layer "F.Cu") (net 8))
 (segment (start 183.1065 87.57) (end 183.645 88.1085) (width 0.2) (layer "F.Cu") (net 8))
 (segment (start 160.49625 104.61625) (end 178.481 86.6315) (width 0.2) (layer "B.Cu") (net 2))
 (segment (start 178.481 86.6315) (end 198.657 86.6315) (width 0.2) (layer "B.Cu") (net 2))
 (segment (start 198.657 86.6315) (end 199.72 85.5685) (width 0.2) (layer "B.Cu") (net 2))
 (segment (start 188.29225 104.61625) (end 199.72 93.1885) (width 0.2) (layer "B.Cu") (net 6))
 (segment (start 179.54625 104.61625) (end 188.29225 104.61625) (width 0.2) (layer "B.Cu") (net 6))
 (segment (start 200.783 91.7115) (end 199.72 90.6485) (width 0.2) (layer "B.Cu") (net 15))
 (segment (start 198.59625 104.61625) (end 200.783 102.4295) (width 0.2) (layer "B.Cu") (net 15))
 (segment (start 200.783 102.4295) (end 200.783 91.7115) (width 0.2) (layer "B.Cu") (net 15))
 (segment (start 201.1385 88.1085) (end 199.72 88.1085) (width 0.2) (layer "B.Cu") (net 16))
 (segment (start 217.64625 104.61625) (end 201.1385 88.1085) (width 0.2) (layer "B.Cu") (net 16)))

